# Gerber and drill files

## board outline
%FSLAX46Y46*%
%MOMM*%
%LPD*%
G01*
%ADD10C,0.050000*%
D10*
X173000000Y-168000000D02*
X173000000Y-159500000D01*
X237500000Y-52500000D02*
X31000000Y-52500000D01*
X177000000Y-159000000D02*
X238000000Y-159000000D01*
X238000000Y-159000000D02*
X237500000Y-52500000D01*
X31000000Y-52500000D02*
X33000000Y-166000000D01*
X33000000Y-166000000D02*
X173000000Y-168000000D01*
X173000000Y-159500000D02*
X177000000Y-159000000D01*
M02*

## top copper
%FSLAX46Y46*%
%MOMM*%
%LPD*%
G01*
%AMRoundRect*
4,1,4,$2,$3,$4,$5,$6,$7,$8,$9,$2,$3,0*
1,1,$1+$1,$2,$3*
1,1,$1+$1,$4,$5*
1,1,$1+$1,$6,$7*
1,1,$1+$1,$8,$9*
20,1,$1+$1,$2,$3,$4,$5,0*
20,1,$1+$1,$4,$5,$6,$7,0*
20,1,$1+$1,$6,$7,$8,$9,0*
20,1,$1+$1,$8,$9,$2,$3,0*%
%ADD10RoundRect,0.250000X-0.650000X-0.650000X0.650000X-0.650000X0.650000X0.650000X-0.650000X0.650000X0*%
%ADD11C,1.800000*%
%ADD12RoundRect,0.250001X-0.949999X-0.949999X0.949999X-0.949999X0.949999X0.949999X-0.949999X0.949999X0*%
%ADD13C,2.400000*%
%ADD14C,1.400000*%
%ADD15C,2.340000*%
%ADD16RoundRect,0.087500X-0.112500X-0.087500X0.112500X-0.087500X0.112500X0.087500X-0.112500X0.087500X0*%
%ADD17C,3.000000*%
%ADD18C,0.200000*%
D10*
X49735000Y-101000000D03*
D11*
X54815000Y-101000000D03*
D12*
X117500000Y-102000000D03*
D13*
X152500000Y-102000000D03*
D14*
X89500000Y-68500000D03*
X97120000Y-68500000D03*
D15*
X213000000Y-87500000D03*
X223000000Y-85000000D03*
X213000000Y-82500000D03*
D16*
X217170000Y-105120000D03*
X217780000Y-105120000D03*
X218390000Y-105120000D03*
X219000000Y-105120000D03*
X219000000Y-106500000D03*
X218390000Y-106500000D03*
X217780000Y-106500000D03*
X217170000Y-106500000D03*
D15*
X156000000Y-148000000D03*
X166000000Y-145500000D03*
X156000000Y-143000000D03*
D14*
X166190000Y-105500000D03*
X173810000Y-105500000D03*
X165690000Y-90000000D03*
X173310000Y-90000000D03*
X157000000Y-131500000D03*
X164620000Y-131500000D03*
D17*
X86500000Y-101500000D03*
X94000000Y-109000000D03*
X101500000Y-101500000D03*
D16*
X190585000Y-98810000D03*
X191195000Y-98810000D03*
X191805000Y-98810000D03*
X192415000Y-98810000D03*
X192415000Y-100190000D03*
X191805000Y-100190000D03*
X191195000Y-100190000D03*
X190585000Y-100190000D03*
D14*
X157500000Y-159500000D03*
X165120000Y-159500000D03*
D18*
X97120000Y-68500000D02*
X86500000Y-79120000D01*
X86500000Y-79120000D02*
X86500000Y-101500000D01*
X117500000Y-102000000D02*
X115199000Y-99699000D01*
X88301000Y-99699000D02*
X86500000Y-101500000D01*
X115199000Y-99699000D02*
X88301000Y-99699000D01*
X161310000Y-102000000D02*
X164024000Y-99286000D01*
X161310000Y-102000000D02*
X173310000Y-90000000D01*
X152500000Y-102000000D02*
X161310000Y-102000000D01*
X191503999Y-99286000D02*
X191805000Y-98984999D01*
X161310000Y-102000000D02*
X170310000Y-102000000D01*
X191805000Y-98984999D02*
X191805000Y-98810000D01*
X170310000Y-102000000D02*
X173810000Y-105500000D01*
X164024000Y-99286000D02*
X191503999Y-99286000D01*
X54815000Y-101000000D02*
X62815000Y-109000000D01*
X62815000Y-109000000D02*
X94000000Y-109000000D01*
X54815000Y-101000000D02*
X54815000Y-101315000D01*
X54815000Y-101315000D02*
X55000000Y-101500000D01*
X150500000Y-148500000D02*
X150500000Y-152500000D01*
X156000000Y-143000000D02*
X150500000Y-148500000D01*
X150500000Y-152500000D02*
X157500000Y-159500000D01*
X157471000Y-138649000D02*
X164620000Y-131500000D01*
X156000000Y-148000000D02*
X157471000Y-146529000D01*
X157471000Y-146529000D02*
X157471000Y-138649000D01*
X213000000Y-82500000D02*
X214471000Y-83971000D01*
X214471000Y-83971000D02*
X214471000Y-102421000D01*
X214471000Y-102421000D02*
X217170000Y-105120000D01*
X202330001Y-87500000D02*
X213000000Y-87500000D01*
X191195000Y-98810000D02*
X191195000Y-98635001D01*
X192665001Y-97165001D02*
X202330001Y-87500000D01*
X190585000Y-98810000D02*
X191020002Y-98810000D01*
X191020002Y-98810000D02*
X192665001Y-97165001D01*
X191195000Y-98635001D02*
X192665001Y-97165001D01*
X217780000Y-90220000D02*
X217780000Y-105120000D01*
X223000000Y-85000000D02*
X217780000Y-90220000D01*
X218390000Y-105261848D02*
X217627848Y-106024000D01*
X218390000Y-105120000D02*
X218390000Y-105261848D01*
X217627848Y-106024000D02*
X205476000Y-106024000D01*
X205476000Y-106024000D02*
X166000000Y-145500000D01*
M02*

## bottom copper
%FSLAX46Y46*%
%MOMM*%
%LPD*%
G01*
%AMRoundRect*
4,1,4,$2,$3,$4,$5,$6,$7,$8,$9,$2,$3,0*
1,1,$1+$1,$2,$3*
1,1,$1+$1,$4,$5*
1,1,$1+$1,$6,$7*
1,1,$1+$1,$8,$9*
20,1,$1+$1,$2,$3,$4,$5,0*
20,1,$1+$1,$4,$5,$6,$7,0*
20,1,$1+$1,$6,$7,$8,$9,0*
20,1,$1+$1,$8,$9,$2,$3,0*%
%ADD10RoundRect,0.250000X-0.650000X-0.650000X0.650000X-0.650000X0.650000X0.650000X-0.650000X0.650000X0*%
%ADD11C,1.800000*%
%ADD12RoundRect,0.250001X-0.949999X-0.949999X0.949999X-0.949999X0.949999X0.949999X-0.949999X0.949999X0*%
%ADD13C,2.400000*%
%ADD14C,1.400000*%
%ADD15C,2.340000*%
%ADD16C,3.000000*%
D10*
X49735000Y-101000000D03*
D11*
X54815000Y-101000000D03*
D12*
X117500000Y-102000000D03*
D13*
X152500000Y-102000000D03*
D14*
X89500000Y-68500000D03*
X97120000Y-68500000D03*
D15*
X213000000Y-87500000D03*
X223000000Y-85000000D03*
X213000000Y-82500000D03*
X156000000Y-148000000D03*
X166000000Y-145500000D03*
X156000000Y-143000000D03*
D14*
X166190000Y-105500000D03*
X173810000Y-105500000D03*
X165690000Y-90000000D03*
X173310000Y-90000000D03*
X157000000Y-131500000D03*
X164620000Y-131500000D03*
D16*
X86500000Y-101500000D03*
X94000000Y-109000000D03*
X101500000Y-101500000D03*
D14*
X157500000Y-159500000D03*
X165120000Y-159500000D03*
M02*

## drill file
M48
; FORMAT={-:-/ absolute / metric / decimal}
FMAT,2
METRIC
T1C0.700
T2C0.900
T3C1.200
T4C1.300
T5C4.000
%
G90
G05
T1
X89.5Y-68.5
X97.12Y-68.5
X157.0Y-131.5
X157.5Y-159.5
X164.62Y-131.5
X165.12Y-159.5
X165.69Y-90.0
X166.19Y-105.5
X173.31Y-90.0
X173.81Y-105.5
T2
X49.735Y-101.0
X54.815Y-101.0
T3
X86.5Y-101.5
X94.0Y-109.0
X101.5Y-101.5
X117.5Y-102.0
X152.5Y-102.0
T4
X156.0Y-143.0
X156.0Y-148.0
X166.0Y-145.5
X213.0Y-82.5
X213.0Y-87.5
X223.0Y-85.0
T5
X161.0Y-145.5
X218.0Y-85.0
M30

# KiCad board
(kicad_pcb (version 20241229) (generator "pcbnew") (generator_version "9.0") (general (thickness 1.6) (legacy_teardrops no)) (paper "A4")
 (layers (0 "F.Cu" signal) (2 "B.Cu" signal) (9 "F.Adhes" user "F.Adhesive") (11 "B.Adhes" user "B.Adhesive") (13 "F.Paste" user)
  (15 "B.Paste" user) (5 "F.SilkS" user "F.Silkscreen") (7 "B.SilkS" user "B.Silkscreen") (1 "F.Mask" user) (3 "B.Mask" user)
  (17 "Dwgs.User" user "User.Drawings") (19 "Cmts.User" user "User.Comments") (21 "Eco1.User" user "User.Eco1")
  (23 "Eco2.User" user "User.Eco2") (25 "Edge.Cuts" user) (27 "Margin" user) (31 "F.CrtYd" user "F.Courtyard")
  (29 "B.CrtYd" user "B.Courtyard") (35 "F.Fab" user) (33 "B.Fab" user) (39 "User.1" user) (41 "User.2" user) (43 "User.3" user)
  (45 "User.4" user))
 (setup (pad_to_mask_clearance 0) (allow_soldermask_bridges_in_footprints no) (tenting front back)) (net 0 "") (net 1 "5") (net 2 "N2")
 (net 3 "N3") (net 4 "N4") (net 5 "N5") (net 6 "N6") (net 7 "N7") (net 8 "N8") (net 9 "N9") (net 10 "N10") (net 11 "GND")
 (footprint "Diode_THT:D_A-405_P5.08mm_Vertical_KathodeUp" (layer "F.Cu") (at 49.735 101)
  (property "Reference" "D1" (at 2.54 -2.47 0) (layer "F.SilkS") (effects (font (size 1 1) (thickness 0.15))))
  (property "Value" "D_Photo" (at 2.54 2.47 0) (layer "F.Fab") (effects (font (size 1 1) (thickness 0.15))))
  (pad "1" thru_hole roundrect (at 0 0) (size 1.8 1.8) (drill 0.9) (layers "*.Cu" "*.Mask") (remove_unused_layers no)
   (roundrect_rratio 0.138889) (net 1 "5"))
  (pad "2" thru_hole circle (at 5.08 0) (size 1.8 1.8) (drill 0.9) (layers "*.Cu" "*.Mask") (remove_unused_layers no) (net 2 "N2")))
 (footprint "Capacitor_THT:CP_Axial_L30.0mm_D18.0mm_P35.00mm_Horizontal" (layer "F.Cu") (at 117.5 102)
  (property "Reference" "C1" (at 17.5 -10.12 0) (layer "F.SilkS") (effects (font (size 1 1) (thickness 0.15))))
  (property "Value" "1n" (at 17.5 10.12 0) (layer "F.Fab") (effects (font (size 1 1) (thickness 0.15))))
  (pad "1" thru_hole roundrect (at 0 0) (size 2.4 2.4) (drill 1.2) (layers "*.Cu" "*.Mask") (remove_unused_layers no)
   (roundrect_rratio 0.104167) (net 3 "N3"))
  (pad "2" thru_hole circle (at 35 0) (size 2.4 2.4) (drill 1.2) (layers "*.Cu" "*.Mask") (remove_unused_layers no) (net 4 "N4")))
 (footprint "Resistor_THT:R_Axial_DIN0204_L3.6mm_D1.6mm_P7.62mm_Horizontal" (layer "F.Cu") (at 89.5 68.5)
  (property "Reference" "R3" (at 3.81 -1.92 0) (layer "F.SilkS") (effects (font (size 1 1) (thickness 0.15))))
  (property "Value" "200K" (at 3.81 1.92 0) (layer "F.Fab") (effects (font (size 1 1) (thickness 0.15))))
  (pad "1" thru_hole circle (at 0 0) (size 1.4 1.4) (drill 0.7) (layers "*.Cu" "*.Mask") (remove_unused_layers no) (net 1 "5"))
  (pad "2" thru_hole circle (at 7.62 0) (size 1.4 1.4) (drill 0.7) (layers "*.Cu" "*.Mask") (remove_unused_layers no) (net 3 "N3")))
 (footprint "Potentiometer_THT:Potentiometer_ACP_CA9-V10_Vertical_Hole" (layer "F.Cu") (at 213 87.5)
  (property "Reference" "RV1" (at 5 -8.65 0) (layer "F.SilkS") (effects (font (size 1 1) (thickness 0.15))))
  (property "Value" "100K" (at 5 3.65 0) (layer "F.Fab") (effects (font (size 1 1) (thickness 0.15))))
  (pad "" np_thru_hole circle (at 5 -2.5) (size 4 4) (drill 4) (layers "*.Cu" "*.Mask"))
  (pad "1" thru_hole circle (at 0 0) (size 2.34 2.34) (drill 1.3) (layers "*.Cu" "*.Mask") (remove_unused_layers no) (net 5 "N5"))
  (pad "2" thru_hole circle (at 10 -2.5) (size 2.34 2.34) (drill 1.3) (layers "*.Cu" "*.Mask") (remove_unused_layers no) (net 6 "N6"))
  (pad "3" thru_hole circle (at 0 -5) (size 2.34 2.34) (drill 1.3) (layers "*.Cu" "*.Mask") (remove_unused_layers no) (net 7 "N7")))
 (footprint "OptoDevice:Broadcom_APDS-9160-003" (layer "F.Cu") (at 218.085 105.81)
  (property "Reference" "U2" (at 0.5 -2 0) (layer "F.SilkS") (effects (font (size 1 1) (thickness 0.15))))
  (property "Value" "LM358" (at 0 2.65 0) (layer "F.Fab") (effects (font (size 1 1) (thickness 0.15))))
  (pad "1" smd roundrect (at -0.915 -0.69) (size 0.4 0.35) (layers "F.Cu" "F.Mask" "F.Paste") (roundrect_rratio 0.25) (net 7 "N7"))
  (pad "2" smd roundrect (at -0.305 -0.69) (size 0.4 0.35) (layers "F.Cu" "F.Mask" "F.Paste") (roundrect_rratio 0.25) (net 6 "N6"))
  (pad "3" smd roundrect (at 0.305 -0.69) (size 0.4 0.35) (layers "F.Cu" "F.Mask" "F.Paste") (roundrect_rratio 0.25) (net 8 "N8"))
  (pad "4" smd roundrect (at 0.915 -0.69) (size 0.4 0.35) (layers "F.Cu" "F.Mask" "F.Paste") (roundrect_rratio 0.25))
  (pad "5" smd roundrect (at 0.915 0.69) (size 0.4 0.35) (layers "F.Cu" "F.Mask" "F.Paste") (roundrect_rratio 0.25))
  (pad "6" smd roundrect (at 0.305 0.69) (size 0.4 0.35) (layers "F.Cu" "F.Mask" "F.Paste") (roundrect_rratio 0.25))
  (pad "7" smd roundrect (at -0.305 0.69) (size 0.4 0.35) (layers "F.Cu" "F.Mask" "F.Paste") (roundrect_rratio 0.25))
  (pad "8" smd roundrect (at -0.915 0.69) (size 0.4 0.35) (layers "F.Cu" "F.Mask" "F.Paste") (roundrect_rratio 0.25)))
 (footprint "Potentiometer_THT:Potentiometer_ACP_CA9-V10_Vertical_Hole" (layer "F.Cu") (at 156 148)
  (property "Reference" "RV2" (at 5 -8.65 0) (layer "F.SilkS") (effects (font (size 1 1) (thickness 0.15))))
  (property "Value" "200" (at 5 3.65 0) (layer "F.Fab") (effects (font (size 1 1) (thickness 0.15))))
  (pad "" np_thru_hole circle (at 5 -2.5) (size 4 4) (drill 4) (layers "*.Cu" "*.Mask"))
  (pad "1" thru_hole circle (at 0 0) (size 2.34 2.34) (drill 1.3) (layers "*.Cu" "*.Mask") (remove_unused_layers no) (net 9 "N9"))
  (pad "2" thru_hole circle (at 10 -2.5) (size 2.34 2.34) (drill 1.3) (layers "*.Cu" "*.Mask") (remove_unused_layers no) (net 8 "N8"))
  (pad "3" thru_hole circle (at 0 -5) (size 2.34 2.34) (drill 1.3) (layers "*.Cu" "*.Mask") (remove_unused_layers no) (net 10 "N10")))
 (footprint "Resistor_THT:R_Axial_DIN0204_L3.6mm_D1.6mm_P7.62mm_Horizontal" (layer "F.Cu") (at 166.19 105.5)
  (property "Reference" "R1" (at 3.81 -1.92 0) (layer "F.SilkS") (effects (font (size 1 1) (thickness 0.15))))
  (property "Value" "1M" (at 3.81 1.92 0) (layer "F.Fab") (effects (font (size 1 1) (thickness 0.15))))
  (pad "1" thru_hole circle (at 0 0) (size 1.4 1.4) (drill 0.7) (layers "*.Cu" "*.Mask") (remove_unused_layers no) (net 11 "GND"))
  (pad "2" thru_hole circle (at 7.62 0) (size 1.4 1.4) (drill 0.7) (layers "*.Cu" "*.Mask") (remove_unused_layers no) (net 4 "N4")))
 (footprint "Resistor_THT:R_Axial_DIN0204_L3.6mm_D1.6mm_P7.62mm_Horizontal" (layer "F.Cu") (at 165.69 90)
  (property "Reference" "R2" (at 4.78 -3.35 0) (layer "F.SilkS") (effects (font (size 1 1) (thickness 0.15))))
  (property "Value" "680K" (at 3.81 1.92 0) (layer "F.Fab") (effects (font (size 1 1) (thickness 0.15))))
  (pad "1" thru_hole circle (at 0 0) (size 1.4 1.4) (drill 0.7) (layers "*.Cu" "*.Mask") (remove_unused_layers no) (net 1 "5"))
  (pad "2" thru_hole circle (at 7.62 0) (size 1.4 1.4) (drill 0.7) (layers "*.Cu" "*.Mask") (remove_unused_layers no) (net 4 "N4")))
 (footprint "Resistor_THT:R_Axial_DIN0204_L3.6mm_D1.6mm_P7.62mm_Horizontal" (layer "F.Cu") (at 157 131.5)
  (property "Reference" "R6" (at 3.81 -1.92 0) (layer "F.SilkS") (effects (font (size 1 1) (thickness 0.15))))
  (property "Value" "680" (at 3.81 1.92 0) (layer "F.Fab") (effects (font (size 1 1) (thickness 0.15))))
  (pad "1" thru_hole circle (at 0 0) (size 1.4 1.4) (drill 0.7) (layers "*.Cu" "*.Mask") (remove_unused_layers no) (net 1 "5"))
  (pad "2" thru_hole circle (at 7.62 0) (size 1.4 1.4) (drill 0.7) (layers "*.Cu" "*.Mask") (remove_unused_layers no) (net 9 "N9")))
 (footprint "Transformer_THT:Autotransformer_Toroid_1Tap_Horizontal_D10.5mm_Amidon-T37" (layer "F.Cu") (at 86.5 101.5)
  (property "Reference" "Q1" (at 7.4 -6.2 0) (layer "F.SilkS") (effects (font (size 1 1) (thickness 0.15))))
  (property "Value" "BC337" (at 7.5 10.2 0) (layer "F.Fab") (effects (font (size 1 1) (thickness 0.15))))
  (pad "1" thru_hole circle (at 0 0) (size 3 3) (drill 1.2) (layers "*.Cu" "*.Mask") (remove_unused_layers no) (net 3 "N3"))
  (pad "2" thru_hole circle (at 7.5 7.5) (size 3 3) (drill 1.2) (layers "*.Cu" "*.Mask") (remove_unused_layers no) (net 2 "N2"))
  (pad "3" thru_hole circle (at 15 0) (size 3 3) (drill 1.2) (layers "*.Cu" "*.Mask") (remove_unused_layers no) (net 11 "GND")))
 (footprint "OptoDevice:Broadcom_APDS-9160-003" (layer "F.Cu") (at 191.5 99.5)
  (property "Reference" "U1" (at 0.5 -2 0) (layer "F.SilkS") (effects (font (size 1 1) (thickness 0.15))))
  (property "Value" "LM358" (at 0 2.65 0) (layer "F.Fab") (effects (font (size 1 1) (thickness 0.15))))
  (pad "1" smd roundrect (at -0.915 -0.69) (size 0.4 0.35) (layers "F.Cu" "F.Mask" "F.Paste") (roundrect_rratio 0.25) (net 5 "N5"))
  (pad "2" smd roundrect (at -0.305 -0.69) (size 0.4 0.35) (layers "F.Cu" "F.Mask" "F.Paste") (roundrect_rratio 0.25) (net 5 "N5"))
  (pad "3" smd roundrect (at 0.305 -0.69) (size 0.4 0.35) (layers "F.Cu" "F.Mask" "F.Paste") (roundrect_rratio 0.25) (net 4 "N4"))
  (pad "4" smd roundrect (at 0.915 -0.69) (size 0.4 0.35) (layers "F.Cu" "F.Mask" "F.Paste") (roundrect_rratio 0.25))
  (pad "5" smd roundrect (at 0.915 0.69) (size 0.4 0.35) (layers "F.Cu" "F.Mask" "F.Paste") (roundrect_rratio 0.25))
  (pad "6" smd roundrect (at 0.305 0.69) (size 0.4 0.35) (layers "F.Cu" "F.Mask" "F.Paste") (roundrect_rratio 0.25))
  (pad "7" smd roundrect (at -0.305 0.69) (size 0.4 0.35) (layers "F.Cu" "F.Mask" "F.Paste") (roundrect_rratio 0.25))
  (pad "8" smd roundrect (at -0.915 0.69) (size 0.4 0.35) (layers "F.Cu" "F.Mask" "F.Paste") (roundrect_rratio 0.25)))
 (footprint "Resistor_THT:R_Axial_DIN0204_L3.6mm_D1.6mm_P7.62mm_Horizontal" (layer "F.Cu") (at 157.5 159.5)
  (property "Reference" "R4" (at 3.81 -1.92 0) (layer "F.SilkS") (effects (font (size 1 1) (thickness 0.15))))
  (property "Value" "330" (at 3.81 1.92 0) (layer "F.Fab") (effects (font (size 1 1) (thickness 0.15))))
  (pad "1" thru_hole circle (at 0 0) (size 1.4 1.4) (drill 0.7) (layers "*.Cu" "*.Mask") (remove_unused_layers no) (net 10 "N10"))
  (pad "2" thru_hole circle (at 7.62 0) (size 1.4 1.4) (drill 0.7) (layers "*.Cu" "*.Mask") (remove_unused_layers no) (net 11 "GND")))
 (gr_line (start 173 168) (end 173 159.5) (stroke (width 0.05) (type default)) (layer "Edge.Cuts"))
 (gr_line (start 237.5 52.5) (end 31 52.5) (stroke (width 0.05) (type default)) (layer "Edge.Cuts"))
 (gr_line (start 177 159) (end 238 159) (stroke (width 0.05) (type default)) (layer "Edge.Cuts"))
 (gr_line (start 238 159) (end 237.5 52.5) (stroke (width 0.05) (type default)) (layer "Edge.Cuts"))
 (gr_line (start 31 52.5) (end 33 166) (stroke (width 0.05) (type default)) (layer "Edge.Cuts"))
 (gr_line (start 33 166) (end 173 168) (stroke (width 0.05) (type default)) (layer "Edge.Cuts"))
 (gr_line (start 173 159.5) (end 177 159) (stroke (width 0.05) (type default)) (layer "Edge.Cuts"))
 (segment (start 97.12 68.5) (end 86.5 79.12) (width 0.2) (layer "F.Cu") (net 3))
 (segment (start 86.5 79.12) (end 86.5 101.5) (width 0.2) (layer "F.Cu") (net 3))
 (segment (start 117.5 102) (end 115.199 99.699) (width 0.2) (layer "F.Cu") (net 3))
 (segment (start 88.301 99.699) (end 86.5 101.5) (width 0.2) (layer "F.Cu") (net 3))
 (segment (start 115.199 99.699) (end 88.301 99.699) (width 0.2) (layer "F.Cu") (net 3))
 (segment (start 161.31 102) (end 164.024 99.286) (width 0.2) (layer "F.Cu") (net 4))
 (segment (start 161.31 102) (end 173.31 90) (width 0.2) (layer "F.Cu") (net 4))
 (segment (start 152.5 102) (end 161.31 102) (width 0.2) (layer "F.Cu") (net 4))
 (segment (start 191.503999 99.286) (end 191.805 98.984999) (width 0.2) (layer "F.Cu") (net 4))
 (segment (start 161.31 102) (end 170.31 102) (width 0.2) (layer "F.Cu") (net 4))
 (segment (start 191.805 98.984999) (end 191.805 98.81) (width 0.2) (layer "F.Cu") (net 4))
 (segment (start 170.31 102) (end 173.81 105.5) (width 0.2) (layer "F.Cu") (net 4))
 (segment (start 164.024 99.286) (end 191.503999 99.286) (width 0.2) (layer "F.Cu") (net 4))
 (segment (start 54.815 101) (end 62.815 109) (width 0.2) (layer "F.Cu") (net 2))
 (segment (start 62.815 109) (end 94 109) (width 0.2) (layer "F.Cu") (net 2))
 (segment (start 54.815 101) (end 54.815 101.315) (width 0.2) (layer "F.Cu") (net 2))
 (segment (start 54.815 101.315) (end 55 101.5) (width 0.2) (layer "F.Cu") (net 2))
 (segment (start 150.5 148.5) (end 150.5 152.5) (width 0.2) (layer "F.Cu") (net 10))
 (segment (start 156 143) (end 150.5 148.5) (width 0.2) (layer "F.Cu") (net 10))
 (segment (start 150.5 152.5) (end 157.5 159.5) (width 0.2) (layer "F.Cu") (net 10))
 (segment (start 157.471 138.649) (end 164.62 131.5) (width 0.2) (layer "F.Cu") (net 9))
 (segment (start 156 148) (end 157.471 146.529) (width 0.2) (layer "F.Cu") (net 9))
 (segment (start 157.471 146.529) (end 157.471 138.649) (width 0.2) (layer "F.Cu") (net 9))
 (segment (start 213 82.5) (end 214.471 83.971) (width 0.2) (layer "F.Cu") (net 7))
 (segment (start 214.471 83.971) (end 214.471 102.421) (width 0.2) (layer "F.Cu") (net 7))
 (segment (start 214.471 102.421) (end 217.17 105.12) (width 0.2) (layer "F.Cu") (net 7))
 (segment (start 202.330001 87.5) (end 213 87.5) (width 0.2) (layer "F.Cu") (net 5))
 (segment (start 191.195 98.81) (end 191.195 98.635001) (width 0.2) (layer "F.Cu") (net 5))
 (segment (start 192.665001 97.165001) (end 202.330001 87.5) (width 0.2) (layer "F.Cu") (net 5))
 (segment (start 190.585 98.81) (end 191.020002 98.81) (width 0.2) (layer "F.Cu") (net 5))
 (segment (start 191.020002 98.81) (end 192.665001 97.165001) (width 0.2) (layer "F.Cu") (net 5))
 (segment (start 191.195 98.635001) (end 192.665001 97.165001) (width 0.2) (layer "F.Cu") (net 5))
 (segment (start 217.78 90.22) (end 217.78 105.12) (width 0.2) (layer "F.Cu") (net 6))
 (segment (start 223 85) (end 217.78 90.22) (width 0.2) (layer "F.Cu") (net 6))
 (segment (start 218.39 105.261848) (end 217.627848 106.024) (width 0.2) (layer "F.Cu") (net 8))
 (segment (start 218.39 105.12) (end 218.39 105.261848) (width 0.2) (layer "F.Cu") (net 8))
 (segment (start 217.627848 106.024) (end 205.476 106.024) (width 0.2) (layer "F.Cu") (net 8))
 (segment (start 205.476 106.024) (end 166 145.5) (width 0.2) (layer "F.Cu") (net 8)))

